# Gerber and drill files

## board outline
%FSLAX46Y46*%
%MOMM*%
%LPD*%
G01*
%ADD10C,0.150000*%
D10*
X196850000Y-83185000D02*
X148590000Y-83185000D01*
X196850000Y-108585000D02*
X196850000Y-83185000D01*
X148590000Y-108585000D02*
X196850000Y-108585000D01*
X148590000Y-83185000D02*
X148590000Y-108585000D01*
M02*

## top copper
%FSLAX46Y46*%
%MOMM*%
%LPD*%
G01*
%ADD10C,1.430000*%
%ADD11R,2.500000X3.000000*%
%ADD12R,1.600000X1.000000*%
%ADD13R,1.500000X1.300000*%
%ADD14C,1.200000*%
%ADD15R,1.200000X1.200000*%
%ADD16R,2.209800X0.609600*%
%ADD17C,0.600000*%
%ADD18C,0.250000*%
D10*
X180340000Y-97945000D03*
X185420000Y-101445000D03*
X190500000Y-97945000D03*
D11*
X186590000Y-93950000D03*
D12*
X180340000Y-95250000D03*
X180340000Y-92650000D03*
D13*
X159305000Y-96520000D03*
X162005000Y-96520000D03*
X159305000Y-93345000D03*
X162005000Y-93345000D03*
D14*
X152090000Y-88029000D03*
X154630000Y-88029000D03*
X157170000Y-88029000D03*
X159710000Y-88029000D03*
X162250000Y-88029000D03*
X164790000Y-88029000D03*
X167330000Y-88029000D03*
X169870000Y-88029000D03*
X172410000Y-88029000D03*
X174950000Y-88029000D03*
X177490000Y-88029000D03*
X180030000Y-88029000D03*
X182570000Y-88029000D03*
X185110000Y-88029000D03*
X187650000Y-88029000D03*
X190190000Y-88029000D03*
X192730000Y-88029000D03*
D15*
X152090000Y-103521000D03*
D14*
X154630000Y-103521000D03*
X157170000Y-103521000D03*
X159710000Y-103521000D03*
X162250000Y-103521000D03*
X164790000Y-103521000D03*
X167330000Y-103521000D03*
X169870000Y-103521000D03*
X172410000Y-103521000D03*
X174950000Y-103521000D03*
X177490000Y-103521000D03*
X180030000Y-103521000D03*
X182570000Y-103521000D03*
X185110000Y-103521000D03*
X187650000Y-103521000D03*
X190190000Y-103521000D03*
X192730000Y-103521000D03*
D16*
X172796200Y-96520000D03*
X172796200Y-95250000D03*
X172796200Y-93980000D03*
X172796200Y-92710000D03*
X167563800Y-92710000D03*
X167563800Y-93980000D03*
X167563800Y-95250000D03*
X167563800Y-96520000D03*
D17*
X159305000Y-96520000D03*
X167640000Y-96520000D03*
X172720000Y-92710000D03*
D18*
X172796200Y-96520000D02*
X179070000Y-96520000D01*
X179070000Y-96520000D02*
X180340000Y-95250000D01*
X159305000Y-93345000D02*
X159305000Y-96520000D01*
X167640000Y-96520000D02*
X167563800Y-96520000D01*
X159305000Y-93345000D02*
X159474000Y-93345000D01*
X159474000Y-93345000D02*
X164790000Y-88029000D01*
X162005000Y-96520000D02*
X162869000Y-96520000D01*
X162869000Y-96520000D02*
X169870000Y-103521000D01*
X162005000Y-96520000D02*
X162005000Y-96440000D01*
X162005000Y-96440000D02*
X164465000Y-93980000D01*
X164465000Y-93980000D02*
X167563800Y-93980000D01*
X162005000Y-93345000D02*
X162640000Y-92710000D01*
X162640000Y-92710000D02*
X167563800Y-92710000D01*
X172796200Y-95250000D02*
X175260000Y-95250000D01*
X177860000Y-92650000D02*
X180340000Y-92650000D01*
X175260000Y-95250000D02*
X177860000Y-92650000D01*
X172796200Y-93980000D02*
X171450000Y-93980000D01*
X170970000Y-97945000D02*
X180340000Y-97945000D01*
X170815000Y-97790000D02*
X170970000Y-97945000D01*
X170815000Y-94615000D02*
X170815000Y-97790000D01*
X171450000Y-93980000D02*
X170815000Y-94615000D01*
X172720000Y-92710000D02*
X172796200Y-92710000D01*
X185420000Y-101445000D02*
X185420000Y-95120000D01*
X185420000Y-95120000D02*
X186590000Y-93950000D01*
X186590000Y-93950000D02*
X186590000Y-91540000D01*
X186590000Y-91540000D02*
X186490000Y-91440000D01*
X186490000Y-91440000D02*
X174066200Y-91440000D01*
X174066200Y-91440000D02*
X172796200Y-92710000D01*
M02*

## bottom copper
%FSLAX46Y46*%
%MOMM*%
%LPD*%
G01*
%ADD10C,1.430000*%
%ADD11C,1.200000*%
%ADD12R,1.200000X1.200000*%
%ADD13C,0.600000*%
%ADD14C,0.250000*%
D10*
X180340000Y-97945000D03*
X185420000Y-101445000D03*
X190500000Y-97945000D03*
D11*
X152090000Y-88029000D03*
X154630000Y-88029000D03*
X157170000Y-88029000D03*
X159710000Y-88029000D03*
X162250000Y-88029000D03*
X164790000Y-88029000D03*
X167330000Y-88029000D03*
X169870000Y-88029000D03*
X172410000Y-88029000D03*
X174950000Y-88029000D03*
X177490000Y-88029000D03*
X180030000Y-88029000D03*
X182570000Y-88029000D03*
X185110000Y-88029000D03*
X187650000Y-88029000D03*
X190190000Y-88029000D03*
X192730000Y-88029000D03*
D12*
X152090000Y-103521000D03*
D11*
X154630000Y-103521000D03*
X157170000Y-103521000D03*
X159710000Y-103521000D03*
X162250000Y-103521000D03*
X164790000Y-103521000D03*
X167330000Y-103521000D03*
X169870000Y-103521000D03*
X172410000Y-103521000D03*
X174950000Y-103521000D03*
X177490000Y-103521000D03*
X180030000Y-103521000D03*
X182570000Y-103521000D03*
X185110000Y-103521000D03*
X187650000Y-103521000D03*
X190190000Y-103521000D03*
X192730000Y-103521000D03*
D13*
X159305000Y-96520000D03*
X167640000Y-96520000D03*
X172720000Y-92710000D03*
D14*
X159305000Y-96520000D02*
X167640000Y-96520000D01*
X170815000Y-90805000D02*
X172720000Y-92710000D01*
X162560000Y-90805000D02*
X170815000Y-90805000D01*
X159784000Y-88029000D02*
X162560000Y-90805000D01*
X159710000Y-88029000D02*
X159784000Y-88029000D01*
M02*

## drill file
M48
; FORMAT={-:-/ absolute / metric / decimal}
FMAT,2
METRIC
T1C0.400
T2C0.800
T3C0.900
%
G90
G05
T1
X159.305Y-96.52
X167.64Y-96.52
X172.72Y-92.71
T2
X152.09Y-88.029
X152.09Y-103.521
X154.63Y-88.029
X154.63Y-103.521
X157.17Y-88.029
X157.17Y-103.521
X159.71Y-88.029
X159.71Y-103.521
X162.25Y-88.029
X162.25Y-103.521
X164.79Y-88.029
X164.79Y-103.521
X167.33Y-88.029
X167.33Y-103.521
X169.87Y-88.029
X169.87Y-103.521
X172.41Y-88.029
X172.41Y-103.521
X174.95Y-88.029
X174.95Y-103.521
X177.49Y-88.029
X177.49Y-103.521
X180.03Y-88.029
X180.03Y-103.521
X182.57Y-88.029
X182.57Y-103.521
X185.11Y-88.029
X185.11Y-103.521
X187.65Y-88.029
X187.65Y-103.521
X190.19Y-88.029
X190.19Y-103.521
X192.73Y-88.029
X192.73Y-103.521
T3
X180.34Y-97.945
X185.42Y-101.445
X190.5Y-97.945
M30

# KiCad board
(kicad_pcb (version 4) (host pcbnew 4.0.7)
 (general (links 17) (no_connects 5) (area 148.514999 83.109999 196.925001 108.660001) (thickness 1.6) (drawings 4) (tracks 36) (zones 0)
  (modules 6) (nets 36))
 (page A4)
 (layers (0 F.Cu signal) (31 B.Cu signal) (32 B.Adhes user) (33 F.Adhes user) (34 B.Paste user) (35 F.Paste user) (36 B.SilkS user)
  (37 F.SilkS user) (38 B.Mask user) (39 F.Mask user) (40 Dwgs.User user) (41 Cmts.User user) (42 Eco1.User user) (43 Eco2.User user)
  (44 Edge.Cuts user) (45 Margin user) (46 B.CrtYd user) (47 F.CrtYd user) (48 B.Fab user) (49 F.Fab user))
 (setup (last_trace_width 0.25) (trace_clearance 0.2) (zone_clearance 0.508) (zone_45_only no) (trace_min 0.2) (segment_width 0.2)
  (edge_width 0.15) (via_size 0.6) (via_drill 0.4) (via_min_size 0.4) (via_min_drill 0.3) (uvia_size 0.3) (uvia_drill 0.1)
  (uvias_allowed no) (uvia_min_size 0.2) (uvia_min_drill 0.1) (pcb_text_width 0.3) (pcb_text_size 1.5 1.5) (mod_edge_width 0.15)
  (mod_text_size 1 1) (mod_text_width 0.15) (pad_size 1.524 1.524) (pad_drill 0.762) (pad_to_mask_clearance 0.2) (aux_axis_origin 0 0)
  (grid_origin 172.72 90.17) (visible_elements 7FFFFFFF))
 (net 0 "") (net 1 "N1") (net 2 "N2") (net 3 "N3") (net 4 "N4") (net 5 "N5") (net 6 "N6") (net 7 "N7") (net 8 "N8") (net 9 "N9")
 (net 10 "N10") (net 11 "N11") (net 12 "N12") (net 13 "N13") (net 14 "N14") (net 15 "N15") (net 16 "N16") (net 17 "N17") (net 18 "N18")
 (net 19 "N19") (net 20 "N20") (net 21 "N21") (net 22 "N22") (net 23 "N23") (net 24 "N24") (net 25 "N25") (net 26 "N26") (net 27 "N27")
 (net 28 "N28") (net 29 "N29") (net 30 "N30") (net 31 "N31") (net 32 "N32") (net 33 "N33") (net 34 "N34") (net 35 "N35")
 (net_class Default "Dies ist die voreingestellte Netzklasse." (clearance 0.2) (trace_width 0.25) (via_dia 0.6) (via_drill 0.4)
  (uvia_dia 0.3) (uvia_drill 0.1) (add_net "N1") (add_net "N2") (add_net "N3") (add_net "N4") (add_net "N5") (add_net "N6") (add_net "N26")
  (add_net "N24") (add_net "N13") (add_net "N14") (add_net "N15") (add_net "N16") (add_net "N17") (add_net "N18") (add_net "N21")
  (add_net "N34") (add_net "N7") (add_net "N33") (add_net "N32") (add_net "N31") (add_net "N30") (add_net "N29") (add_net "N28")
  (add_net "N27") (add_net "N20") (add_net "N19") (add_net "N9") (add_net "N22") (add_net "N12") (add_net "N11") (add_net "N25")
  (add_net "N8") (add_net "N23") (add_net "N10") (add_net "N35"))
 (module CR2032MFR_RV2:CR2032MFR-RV (layer F.Cu) (at 185.42 99.695)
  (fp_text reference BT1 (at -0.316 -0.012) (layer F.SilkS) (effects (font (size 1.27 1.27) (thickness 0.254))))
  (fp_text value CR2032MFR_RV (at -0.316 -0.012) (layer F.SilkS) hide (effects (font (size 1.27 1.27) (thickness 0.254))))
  (pad 1 thru_hole circle (at -5.08 -1.75 90) (size 1.43 1.43) (drill 0.9) (layers *.Cu *.Mask F.SilkS) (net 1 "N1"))
  (pad 2 thru_hole circle (at 0 1.75 90) (size 1.43 1.43) (drill 0.9) (layers *.Cu *.Mask F.SilkS) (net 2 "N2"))
  (pad 3 thru_hole circle (at 5.08 -1.75 90) (size 1.43 1.43) (drill 0.9) (layers *.Cu *.Mask F.SilkS) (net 1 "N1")))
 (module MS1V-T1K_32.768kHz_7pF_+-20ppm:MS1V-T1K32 (layer F.Cu) (at 180.34 95.25 180)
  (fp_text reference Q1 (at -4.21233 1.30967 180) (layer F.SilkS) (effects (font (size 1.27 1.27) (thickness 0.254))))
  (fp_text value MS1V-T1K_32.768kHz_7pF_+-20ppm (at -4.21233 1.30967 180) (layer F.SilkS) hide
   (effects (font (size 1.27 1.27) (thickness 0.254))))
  (pad 1 smd rect (at -6.25 1.3 180) (size 2.5 3) (layers F.Cu F.Paste F.Mask) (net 2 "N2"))
  (pad 2 smd rect (at 0 0 270) (size 1 1.6) (layers F.Cu F.Paste F.Mask) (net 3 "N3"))
  (pad 3 smd rect (at 0 2.6 270) (size 1 1.6) (layers F.Cu F.Paste F.Mask) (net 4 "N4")))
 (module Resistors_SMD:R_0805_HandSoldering (layer F.Cu) (at 160.655 96.52)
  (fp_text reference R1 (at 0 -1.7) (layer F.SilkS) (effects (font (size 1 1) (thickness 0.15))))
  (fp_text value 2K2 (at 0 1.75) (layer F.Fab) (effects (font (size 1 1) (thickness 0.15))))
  (pad 1 smd rect (at -1.35 0) (size 1.5 1.3) (layers F.Cu F.Paste F.Mask) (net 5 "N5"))
  (pad 2 smd rect (at 1.35 0) (size 1.5 1.3) (layers F.Cu F.Paste F.Mask) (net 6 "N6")))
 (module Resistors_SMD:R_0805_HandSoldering (layer F.Cu) (at 160.655 93.345)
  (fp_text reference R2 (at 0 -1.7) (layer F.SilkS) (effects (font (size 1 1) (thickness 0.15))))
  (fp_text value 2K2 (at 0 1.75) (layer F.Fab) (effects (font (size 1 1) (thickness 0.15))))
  (pad 1 smd rect (at -1.35 0) (size 1.5 1.3) (layers F.Cu F.Paste F.Mask) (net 5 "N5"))
  (pad 2 smd rect (at 1.35 0) (size 1.5 1.3) (layers F.Cu F.Paste F.Mask) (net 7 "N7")))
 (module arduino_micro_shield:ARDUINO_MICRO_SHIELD (layer F.Cu) (at 148.59 104.775)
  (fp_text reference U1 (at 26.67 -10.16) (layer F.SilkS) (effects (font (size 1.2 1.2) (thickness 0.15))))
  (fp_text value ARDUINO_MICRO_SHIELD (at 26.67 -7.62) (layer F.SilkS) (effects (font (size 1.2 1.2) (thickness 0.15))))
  (pad SCK thru_hole circle (at 3.5 -16.746) (size 1.2 1.2) (drill 0.8) (layers *.Cu *.Mask F.SilkS) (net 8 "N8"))
  (pad MI thru_hole circle (at 6.04 -16.746) (size 1.2 1.2) (drill 0.8) (layers *.Cu *.Mask F.SilkS) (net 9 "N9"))
  (pad VI thru_hole circle (at 8.58 -16.746) (size 1.2 1.2) (drill 0.8) (layers *.Cu *.Mask F.SilkS) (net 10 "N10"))
  (pad GND thru_hole circle (at 11.12 -16.746) (size 1.2 1.2) (drill 0.8) (layers *.Cu *.Mask F.SilkS) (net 2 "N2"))
  (pad RST thru_hole circle (at 13.66 -16.746) (size 1.2 1.2) (drill 0.8) (layers *.Cu *.Mask F.SilkS) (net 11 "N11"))
  (pad 5V thru_hole circle (at 16.2 -16.746) (size 1.2 1.2) (drill 0.8) (layers *.Cu *.Mask F.SilkS) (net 5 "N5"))
  (pad NC thru_hole circle (at 18.74 -16.746) (size 1.2 1.2) (drill 0.8) (layers *.Cu *.Mask F.SilkS) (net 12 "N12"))
  (pad NC thru_hole circle (at 21.28 -16.746) (size 1.2 1.2) (drill 0.8) (layers *.Cu *.Mask F.SilkS) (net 12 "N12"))
  (pad A5 thru_hole circle (at 23.82 -16.746) (size 1.2 1.2) (drill 0.8) (layers *.Cu *.Mask F.SilkS) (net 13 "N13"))
  (pad A4 thru_hole circle (at 26.36 -16.746) (size 1.2 1.2) (drill 0.8) (layers *.Cu *.Mask F.SilkS) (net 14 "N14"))
  (pad A3 thru_hole circle (at 28.9 -16.746) (size 1.2 1.2) (drill 0.8) (layers *.Cu *.Mask F.SilkS) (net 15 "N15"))
  (pad A2 thru_hole circle (at 31.44 -16.746) (size 1.2 1.2) (drill 0.8) (layers *.Cu *.Mask F.SilkS) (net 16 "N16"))
  (pad A1 thru_hole circle (at 33.98 -16.746) (size 1.2 1.2) (drill 0.8) (layers *.Cu *.Mask F.SilkS) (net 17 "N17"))
  (pad A0 thru_hole circle (at 36.52 -16.746) (size 1.2 1.2) (drill 0.8) (layers *.Cu *.Mask F.SilkS) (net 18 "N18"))
  (pad AREF thru_hole circle (at 39.06 -16.746) (size 1.2 1.2) (drill 0.8) (layers *.Cu *.Mask F.SilkS) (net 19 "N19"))
  (pad 3.3V thru_hole circle (at 41.6 -16.746) (size 1.2 1.2) (drill 0.8) (layers *.Cu *.Mask F.SilkS) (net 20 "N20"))
  (pad 13 thru_hole circle (at 44.14 -16.746) (size 1.2 1.2) (drill 0.8) (layers *.Cu *.Mask F.SilkS) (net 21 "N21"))
  (pad MO thru_hole rect (at 3.5 -1.254) (size 1.2 1.2) (drill 0.8) (layers *.Cu *.Mask F.SilkS) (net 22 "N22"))
  (pad SS thru_hole circle (at 6.04 -1.254) (size 1.2 1.2) (drill 0.8) (layers *.Cu *.Mask F.SilkS) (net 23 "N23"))
  (pad TX thru_hole circle (at 8.58 -1.254) (size 1.2 1.2) (drill 0.8) (layers *.Cu *.Mask F.SilkS) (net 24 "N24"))
  (pad RX thru_hole circle (at 11.12 -1.254) (size 1.2 1.2) (drill 0.8) (layers *.Cu *.Mask F.SilkS) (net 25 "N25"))
  (pad RST thru_hole circle (at 13.66 -1.254) (size 1.2 1.2) (drill 0.8) (layers *.Cu *.Mask F.SilkS) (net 11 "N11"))
  (pad GND thru_hole circle (at 16.2 -1.254) (size 1.2 1.2) (drill 0.8) (layers *.Cu *.Mask F.SilkS) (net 2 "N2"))
  (pad 2 thru_hole circle (at 18.74 -1.254) (size 1.2 1.2) (drill 0.8) (layers *.Cu *.Mask F.SilkS) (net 7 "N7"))
  (pad 3 thru_hole circle (at 21.28 -1.254) (size 1.2 1.2) (drill 0.8) (layers *.Cu *.Mask F.SilkS) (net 6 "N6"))
  (pad 4 thru_hole circle (at 23.82 -1.254) (size 1.2 1.2) (drill 0.8) (layers *.Cu *.Mask F.SilkS) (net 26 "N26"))
  (pad 5 thru_hole circle (at 26.36 -1.254) (size 1.2 1.2) (drill 0.8) (layers *.Cu *.Mask F.SilkS) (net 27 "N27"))
  (pad 6 thru_hole circle (at 28.9 -1.254) (size 1.2 1.2) (drill 0.8) (layers *.Cu *.Mask F.SilkS) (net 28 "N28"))
  (pad 7 thru_hole circle (at 31.44 -1.254) (size 1.2 1.2) (drill 0.8) (layers *.Cu *.Mask F.SilkS) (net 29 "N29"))
  (pad 8 thru_hole circle (at 33.98 -1.254) (size 1.2 1.2) (drill 0.8) (layers *.Cu *.Mask F.SilkS) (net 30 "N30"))
  (pad 9 thru_hole circle (at 36.52 -1.254) (size 1.2 1.2) (drill 0.8) (layers *.Cu *.Mask F.SilkS) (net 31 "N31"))
  (pad 10 thru_hole circle (at 39.06 -1.254) (size 1.2 1.2) (drill 0.8) (layers *.Cu *.Mask F.SilkS) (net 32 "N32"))
  (pad 11 thru_hole circle (at 41.6 -1.254) (size 1.2 1.2) (drill 0.8) (layers *.Cu *.Mask F.SilkS) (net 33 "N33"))
  (pad 12 thru_hole circle (at 44.14 -1.254) (size 1.2 1.2) (drill 0.8) (layers *.Cu *.Mask F.SilkS) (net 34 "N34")))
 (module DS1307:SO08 (layer F.Cu) (at 170.18 94.615 90)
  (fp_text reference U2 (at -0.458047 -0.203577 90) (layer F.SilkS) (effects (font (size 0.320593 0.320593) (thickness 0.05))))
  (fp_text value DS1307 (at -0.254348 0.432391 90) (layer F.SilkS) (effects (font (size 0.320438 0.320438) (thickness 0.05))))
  (pad 1 smd rect (at -1.905 2.6162 90) (size 0.6096 2.2098) (layers F.Cu F.Paste F.Mask) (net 3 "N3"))
  (pad 2 smd rect (at -0.635 2.6162 90) (size 0.6096 2.2098) (layers F.Cu F.Paste F.Mask) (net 4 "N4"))
  (pad 3 smd rect (at 0.635 2.6162 90) (size 0.6096 2.2098) (layers F.Cu F.Paste F.Mask) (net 1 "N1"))
  (pad 4 smd rect (at 1.905 2.6162 90) (size 0.6096 2.2098) (layers F.Cu F.Paste F.Mask) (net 2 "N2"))
  (pad 5 smd rect (at 1.905 -2.6162 90) (size 0.6096 2.2098) (layers F.Cu F.Paste F.Mask) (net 7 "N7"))
  (pad 6 smd rect (at 0.635 -2.6162 90) (size 0.6096 2.2098) (layers F.Cu F.Paste F.Mask) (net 6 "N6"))
  (pad 7 smd rect (at -0.635 -2.6162 90) (size 0.6096 2.2098) (layers F.Cu F.Paste F.Mask) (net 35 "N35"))
  (pad 8 smd rect (at -1.905 -2.6162 90) (size 0.6096 2.2098) (layers F.Cu F.Paste F.Mask) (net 5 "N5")))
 (gr_line (start 196.85 83.185) (end 148.59 83.185) (angle 90) (layer Edge.Cuts) (width 0.15))
 (gr_line (start 196.85 108.585) (end 196.85 83.185) (angle 90) (layer Edge.Cuts) (width 0.15))
 (gr_line (start 148.59 108.585) (end 196.85 108.585) (angle 90) (layer Edge.Cuts) (width 0.15))
 (gr_line (start 148.59 83.185) (end 148.59 108.585) (angle 90) (layer Edge.Cuts) (width 0.15))
 (segment (start 172.7962 96.52) (end 179.07 96.52) (width 0.25) (layer F.Cu) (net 3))
 (segment (start 179.07 96.52) (end 180.34 95.25) (width 0.25) (layer F.Cu) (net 3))
 (via (at 159.305 96.52) (size 0.6) (drill 0.4) (layers F.Cu B.Cu) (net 5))
 (segment (start 159.305 93.345) (end 159.305 96.52) (width 0.25) (layer F.Cu) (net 5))
 (segment (start 167.64 96.52) (end 167.5638 96.52) (width 0.25) (layer F.Cu) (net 5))
 (via (at 167.64 96.52) (size 0.6) (drill 0.4) (layers F.Cu B.Cu) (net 5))
 (segment (start 159.305 96.52) (end 167.64 96.52) (width 0.25) (layer B.Cu) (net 5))
 (segment (start 159.305 93.345) (end 159.474 93.345) (width 0.25) (layer F.Cu) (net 5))
 (segment (start 159.474 93.345) (end 164.79 88.029) (width 0.25) (layer F.Cu) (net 5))
 (segment (start 162.005 96.52) (end 162.869 96.52) (width 0.25) (layer F.Cu) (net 6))
 (segment (start 162.869 96.52) (end 169.87 103.521) (width 0.25) (layer F.Cu) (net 6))
 (segment (start 162.005 96.52) (end 162.005 96.44) (width 0.25) (layer F.Cu) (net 6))
 (segment (start 162.005 96.44) (end 164.465 93.98) (width 0.25) (layer F.Cu) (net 6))
 (segment (start 164.465 93.98) (end 167.5638 93.98) (width 0.25) (layer F.Cu) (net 6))
 (segment (start 162.005 93.345) (end 162.64 92.71) (width 0.25) (layer F.Cu) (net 7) (status C00000))
 (segment (start 162.64 92.71) (end 167.5638 92.71) (width 0.25) (layer F.Cu) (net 7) (status C00000))
 (segment (start 172.7962 95.25) (end 175.26 95.25) (width 0.25) (layer F.Cu) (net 4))
 (segment (start 177.86 92.65) (end 180.34 92.65) (width 0.25) (layer F.Cu) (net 4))
 (segment (start 175.26 95.25) (end 177.86 92.65) (width 0.25) (layer F.Cu) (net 4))
 (segment (start 172.7962 93.98) (end 171.45 93.98) (width 0.25) (layer F.Cu) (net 1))
 (segment (start 170.97 97.945) (end 180.34 97.945) (width 0.25) (layer F.Cu) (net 1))
 (segment (start 170.815 97.79) (end 170.97 97.945) (width 0.25) (layer F.Cu) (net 1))
 (segment (start 170.815 94.615) (end 170.815 97.79) (width 0.25) (layer F.Cu) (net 1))
 (segment (start 171.45 93.98) (end 170.815 94.615) (width 0.25) (layer F.Cu) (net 1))
 (segment (start 172.72 92.71) (end 172.7962 92.71) (width 0.25) (layer F.Cu) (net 2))
 (via (at 172.72 92.71) (size 0.6) (drill 0.4) (layers F.Cu B.Cu) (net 2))
 (segment (start 170.815 90.805) (end 172.72 92.71) (width 0.25) (layer B.Cu) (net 2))
 (segment (start 162.56 90.805) (end 170.815 90.805) (width 0.25) (layer B.Cu) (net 2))
 (segment (start 159.784 88.029) (end 162.56 90.805) (width 0.25) (layer B.Cu) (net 2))
 (segment (start 159.71 88.029) (end 159.784 88.029) (width 0.25) (layer B.Cu) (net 2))
 (segment (start 185.42 101.445) (end 185.42 95.12) (width 0.25) (layer F.Cu) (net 2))
 (segment (start 185.42 95.12) (end 186.59 93.95) (width 0.25) (layer F.Cu) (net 2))
 (segment (start 186.59 93.95) (end 186.59 91.54) (width 0.25) (layer F.Cu) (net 2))
 (segment (start 186.59 91.54) (end 186.49 91.44) (width 0.25) (layer F.Cu) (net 2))
 (segment (start 186.49 91.44) (end 174.0662 91.44) (width 0.25) (layer F.Cu) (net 2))
 (segment (start 174.0662 91.44) (end 172.7962 92.71) (width 0.25) (layer F.Cu) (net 2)))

